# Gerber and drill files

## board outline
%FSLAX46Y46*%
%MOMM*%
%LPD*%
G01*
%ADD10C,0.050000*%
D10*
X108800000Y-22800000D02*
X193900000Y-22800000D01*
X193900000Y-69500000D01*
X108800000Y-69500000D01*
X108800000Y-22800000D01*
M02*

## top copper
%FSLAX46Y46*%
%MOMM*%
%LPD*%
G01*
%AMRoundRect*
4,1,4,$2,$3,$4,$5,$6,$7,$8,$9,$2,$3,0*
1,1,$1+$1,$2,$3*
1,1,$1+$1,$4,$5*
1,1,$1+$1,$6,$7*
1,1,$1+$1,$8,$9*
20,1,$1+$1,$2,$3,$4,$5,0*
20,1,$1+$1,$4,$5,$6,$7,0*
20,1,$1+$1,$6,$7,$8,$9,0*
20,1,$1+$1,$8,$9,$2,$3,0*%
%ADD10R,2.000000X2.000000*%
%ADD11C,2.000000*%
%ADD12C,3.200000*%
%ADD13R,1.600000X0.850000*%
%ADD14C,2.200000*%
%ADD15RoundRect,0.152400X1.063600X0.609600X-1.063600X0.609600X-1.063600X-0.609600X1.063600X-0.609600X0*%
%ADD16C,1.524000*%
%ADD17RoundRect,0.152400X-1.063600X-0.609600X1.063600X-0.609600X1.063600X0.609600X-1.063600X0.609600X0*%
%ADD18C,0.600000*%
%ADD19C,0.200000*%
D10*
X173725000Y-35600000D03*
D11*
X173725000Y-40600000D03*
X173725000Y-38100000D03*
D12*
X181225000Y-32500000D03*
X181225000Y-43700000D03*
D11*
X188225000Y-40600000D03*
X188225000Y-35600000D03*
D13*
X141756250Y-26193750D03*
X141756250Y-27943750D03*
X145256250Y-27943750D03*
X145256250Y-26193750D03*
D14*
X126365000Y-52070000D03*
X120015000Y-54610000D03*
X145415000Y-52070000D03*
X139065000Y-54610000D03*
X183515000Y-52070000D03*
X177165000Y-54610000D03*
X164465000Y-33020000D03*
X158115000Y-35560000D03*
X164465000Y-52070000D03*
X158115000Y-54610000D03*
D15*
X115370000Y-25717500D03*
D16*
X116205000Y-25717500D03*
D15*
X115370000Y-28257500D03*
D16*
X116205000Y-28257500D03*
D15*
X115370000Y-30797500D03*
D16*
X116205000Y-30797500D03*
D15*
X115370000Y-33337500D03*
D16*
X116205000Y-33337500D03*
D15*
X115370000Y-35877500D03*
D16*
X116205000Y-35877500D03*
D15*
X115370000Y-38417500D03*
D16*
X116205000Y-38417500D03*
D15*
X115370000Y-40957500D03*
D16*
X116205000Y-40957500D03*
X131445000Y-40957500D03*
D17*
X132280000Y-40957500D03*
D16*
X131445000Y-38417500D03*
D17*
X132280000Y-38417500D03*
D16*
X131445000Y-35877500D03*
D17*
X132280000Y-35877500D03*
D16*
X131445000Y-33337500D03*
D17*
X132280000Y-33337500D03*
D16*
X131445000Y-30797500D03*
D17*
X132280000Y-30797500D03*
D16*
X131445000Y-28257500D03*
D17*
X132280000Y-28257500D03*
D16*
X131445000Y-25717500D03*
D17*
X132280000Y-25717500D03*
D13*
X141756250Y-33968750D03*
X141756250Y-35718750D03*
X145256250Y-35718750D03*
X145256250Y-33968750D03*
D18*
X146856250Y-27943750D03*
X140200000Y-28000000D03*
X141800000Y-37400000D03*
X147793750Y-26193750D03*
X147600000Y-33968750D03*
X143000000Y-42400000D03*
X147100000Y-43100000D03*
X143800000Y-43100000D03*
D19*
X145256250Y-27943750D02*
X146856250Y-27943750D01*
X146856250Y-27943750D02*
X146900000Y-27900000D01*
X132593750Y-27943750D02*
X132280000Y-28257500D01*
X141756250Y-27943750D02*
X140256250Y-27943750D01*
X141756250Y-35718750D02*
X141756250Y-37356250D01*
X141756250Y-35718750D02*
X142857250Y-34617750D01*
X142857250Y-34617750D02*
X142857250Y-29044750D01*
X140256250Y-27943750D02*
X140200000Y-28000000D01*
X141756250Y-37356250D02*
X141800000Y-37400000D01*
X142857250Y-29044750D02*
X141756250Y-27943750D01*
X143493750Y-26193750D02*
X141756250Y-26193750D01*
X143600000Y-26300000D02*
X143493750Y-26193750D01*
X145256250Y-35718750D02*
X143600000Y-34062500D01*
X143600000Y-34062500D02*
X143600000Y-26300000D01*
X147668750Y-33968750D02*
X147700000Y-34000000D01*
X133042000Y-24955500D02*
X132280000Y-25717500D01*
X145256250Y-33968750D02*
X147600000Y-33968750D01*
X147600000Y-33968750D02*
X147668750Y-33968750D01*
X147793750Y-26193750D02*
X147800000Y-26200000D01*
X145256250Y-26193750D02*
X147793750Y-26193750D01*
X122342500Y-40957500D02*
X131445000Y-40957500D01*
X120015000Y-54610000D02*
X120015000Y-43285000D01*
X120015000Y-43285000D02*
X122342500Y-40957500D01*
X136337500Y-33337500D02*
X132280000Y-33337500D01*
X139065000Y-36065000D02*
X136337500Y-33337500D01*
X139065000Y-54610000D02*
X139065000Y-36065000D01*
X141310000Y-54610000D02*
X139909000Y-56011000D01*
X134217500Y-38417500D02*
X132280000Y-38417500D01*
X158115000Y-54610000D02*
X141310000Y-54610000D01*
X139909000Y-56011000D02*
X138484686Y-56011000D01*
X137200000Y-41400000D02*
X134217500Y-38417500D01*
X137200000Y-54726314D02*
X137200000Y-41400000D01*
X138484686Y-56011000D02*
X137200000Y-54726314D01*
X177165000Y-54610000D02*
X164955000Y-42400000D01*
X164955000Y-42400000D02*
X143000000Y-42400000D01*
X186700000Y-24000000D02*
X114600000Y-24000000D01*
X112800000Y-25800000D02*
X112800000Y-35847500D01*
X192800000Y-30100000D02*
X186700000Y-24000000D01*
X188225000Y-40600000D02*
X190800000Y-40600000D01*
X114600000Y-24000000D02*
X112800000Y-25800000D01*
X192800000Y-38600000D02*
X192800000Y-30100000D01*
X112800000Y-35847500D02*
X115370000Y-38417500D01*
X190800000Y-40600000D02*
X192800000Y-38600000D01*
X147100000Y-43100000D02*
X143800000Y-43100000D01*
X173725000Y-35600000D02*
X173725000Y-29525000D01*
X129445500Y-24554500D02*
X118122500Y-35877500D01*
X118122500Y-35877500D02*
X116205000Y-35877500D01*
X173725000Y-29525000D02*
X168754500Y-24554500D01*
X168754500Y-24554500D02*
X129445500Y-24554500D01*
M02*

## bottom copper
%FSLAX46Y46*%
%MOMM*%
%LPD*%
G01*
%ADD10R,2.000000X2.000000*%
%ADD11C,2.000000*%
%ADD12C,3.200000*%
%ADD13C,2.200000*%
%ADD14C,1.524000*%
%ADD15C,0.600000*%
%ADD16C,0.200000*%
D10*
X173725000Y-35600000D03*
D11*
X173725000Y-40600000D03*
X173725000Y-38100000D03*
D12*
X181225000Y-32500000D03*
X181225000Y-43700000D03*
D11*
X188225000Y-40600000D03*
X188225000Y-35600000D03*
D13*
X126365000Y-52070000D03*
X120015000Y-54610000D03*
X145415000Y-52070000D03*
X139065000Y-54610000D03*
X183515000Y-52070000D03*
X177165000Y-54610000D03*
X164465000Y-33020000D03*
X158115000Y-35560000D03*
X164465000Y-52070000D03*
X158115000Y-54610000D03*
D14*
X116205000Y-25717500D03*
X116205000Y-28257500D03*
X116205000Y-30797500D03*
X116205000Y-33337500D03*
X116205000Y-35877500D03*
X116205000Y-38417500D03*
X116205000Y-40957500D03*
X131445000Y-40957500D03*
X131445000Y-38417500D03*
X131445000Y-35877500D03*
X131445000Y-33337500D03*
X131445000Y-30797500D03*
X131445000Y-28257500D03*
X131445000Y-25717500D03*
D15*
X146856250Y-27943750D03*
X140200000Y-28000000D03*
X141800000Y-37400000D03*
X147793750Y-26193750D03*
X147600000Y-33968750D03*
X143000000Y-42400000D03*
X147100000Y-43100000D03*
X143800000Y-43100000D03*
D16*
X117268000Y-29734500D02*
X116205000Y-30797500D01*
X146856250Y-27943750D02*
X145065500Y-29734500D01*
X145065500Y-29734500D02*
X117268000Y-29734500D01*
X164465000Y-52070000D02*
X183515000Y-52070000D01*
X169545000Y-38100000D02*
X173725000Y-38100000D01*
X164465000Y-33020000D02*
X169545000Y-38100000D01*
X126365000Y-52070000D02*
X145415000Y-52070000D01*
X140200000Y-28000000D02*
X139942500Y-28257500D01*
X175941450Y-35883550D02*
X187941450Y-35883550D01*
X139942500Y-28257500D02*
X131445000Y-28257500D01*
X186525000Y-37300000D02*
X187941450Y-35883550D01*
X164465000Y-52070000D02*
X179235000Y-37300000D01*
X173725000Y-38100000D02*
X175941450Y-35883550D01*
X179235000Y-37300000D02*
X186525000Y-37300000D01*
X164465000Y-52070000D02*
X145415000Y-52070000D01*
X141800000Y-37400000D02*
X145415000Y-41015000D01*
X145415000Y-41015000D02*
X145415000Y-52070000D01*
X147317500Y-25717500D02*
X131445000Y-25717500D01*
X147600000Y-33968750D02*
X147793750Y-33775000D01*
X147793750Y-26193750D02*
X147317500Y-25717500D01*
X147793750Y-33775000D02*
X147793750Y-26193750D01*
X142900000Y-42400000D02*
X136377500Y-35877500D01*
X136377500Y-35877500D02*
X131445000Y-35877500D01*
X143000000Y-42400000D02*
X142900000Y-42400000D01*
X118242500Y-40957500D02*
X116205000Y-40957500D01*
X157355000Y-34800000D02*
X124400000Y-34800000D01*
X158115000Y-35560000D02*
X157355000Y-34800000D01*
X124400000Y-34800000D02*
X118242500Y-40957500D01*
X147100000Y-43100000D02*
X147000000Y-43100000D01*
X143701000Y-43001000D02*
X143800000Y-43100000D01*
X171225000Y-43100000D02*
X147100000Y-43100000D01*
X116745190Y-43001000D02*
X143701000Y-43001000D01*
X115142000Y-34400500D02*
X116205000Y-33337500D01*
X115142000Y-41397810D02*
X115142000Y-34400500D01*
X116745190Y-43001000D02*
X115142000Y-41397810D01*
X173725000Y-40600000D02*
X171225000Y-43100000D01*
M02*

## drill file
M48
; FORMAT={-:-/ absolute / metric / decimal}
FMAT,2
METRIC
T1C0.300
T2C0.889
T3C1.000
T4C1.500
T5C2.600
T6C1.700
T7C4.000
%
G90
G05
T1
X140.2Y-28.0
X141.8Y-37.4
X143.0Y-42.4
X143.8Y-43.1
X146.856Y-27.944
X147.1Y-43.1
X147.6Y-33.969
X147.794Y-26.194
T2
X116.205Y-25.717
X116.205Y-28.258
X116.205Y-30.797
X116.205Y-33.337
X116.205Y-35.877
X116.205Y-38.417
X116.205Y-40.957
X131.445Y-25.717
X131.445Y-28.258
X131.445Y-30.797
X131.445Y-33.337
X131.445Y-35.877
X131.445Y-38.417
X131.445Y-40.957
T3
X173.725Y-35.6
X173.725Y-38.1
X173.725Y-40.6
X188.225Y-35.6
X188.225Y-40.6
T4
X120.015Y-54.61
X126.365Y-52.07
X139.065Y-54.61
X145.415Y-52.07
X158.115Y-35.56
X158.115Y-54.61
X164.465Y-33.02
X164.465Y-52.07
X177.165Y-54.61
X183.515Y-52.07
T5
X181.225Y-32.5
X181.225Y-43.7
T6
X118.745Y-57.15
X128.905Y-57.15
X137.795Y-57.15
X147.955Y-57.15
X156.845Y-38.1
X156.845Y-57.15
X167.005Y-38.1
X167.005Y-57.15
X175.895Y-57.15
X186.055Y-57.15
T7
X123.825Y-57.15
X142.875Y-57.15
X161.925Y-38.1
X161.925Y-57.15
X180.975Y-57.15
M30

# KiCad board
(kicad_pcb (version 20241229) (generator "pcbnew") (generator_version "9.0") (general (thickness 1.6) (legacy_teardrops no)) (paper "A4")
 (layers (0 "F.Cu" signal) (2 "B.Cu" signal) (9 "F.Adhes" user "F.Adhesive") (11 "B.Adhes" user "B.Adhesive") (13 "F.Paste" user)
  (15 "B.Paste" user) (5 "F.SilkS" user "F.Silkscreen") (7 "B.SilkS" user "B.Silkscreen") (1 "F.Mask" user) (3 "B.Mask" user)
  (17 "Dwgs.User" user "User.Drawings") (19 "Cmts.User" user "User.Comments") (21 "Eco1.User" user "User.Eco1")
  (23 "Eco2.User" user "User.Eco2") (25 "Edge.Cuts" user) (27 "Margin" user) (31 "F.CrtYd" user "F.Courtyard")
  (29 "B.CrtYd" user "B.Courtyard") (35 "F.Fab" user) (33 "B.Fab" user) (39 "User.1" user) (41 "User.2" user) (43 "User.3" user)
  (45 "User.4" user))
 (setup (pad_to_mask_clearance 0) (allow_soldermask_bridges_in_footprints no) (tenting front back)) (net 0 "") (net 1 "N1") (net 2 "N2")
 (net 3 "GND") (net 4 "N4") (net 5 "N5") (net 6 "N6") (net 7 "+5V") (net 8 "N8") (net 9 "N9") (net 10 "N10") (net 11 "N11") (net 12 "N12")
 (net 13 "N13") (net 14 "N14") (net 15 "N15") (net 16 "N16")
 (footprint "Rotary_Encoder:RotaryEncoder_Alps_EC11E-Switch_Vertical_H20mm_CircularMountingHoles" (layer "F.Cu") (at 173.725 35.6)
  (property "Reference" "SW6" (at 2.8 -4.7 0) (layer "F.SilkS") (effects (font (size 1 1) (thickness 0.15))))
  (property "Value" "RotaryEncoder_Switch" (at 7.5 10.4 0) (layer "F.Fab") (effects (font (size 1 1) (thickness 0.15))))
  (pad "A" thru_hole rect (at 0 0) (size 2 2) (drill 1) (layers "*.Cu" "*.Mask") (remove_unused_layers no) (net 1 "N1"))
  (pad "B" thru_hole circle (at 0 5) (size 2 2) (drill 1) (layers "*.Cu" "*.Mask") (remove_unused_layers no) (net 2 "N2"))
  (pad "C" thru_hole circle (at 0 2.5) (size 2 2) (drill 1) (layers "*.Cu" "*.Mask") (remove_unused_layers no) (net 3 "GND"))
  (pad "MP" thru_hole circle (at 7.5 -3.1) (size 3.2 3.2) (drill 2.6) (layers "*.Cu" "*.Mask") (remove_unused_layers no))
  (pad "MP" thru_hole circle (at 7.5 8.1) (size 3.2 3.2) (drill 2.6) (layers "*.Cu" "*.Mask") (remove_unused_layers no))
  (pad "S1" thru_hole circle (at 14.5 5) (size 2 2) (drill 1) (layers "*.Cu" "*.Mask") (remove_unused_layers no) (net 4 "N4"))
  (pad "S2" thru_hole circle (at 14.5 0) (size 2 2) (drill 1) (layers "*.Cu" "*.Mask") (remove_unused_layers no) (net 3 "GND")))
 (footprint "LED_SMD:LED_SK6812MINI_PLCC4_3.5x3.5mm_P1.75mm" (layer "F.Cu") (at 143.50625 27.06875)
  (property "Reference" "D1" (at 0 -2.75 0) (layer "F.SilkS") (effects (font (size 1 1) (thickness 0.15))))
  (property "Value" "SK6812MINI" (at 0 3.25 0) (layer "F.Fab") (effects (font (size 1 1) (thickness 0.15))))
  (pad "1" smd rect (at -1.75 -0.875) (size 1.6 0.85) (layers "F.Cu" "F.Mask" "F.Paste") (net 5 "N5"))
  (pad "2" smd rect (at -1.75 0.875) (size 1.6 0.85) (layers "F.Cu" "F.Mask" "F.Paste") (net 3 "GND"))
  (pad "3" smd rect (at 1.75 0.875) (size 1.6 0.85) (layers "F.Cu" "F.Mask" "F.Paste") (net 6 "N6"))
  (pad "4" smd rect (at 1.75 -0.875) (size 1.6 0.85) (layers "F.Cu" "F.Mask" "F.Paste") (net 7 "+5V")))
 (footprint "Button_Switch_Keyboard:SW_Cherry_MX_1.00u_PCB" (layer "F.Cu") (at 126.365 52.07)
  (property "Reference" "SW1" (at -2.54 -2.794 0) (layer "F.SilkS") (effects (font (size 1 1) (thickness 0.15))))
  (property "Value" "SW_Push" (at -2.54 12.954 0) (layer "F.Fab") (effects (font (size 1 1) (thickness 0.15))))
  (pad "" np_thru_hole circle (at -7.62 5.08) (size 1.7 1.7) (drill 1.7) (layers "*.Cu" "*.Mask"))
  (pad "" np_thru_hole circle (at -2.54 5.08) (size 4 4) (drill 4) (layers "*.Cu" "*.Mask"))
  (pad "" np_thru_hole circle (at 2.54 5.08) (size 1.7 1.7) (drill 1.7) (layers "*.Cu" "*.Mask"))
  (pad "1" thru_hole circle (at 0 0) (size 2.2 2.2) (drill 1.5) (layers "*.Cu" "*.Mask") (remove_unused_layers no) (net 3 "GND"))
  (pad "2" thru_hole circle (at -6.35 2.54) (size 2.2 2.2) (drill 1.5) (layers "*.Cu" "*.Mask") (remove_unused_layers no) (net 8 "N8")))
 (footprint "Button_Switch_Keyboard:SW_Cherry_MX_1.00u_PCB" (layer "F.Cu") (at 145.415 52.07)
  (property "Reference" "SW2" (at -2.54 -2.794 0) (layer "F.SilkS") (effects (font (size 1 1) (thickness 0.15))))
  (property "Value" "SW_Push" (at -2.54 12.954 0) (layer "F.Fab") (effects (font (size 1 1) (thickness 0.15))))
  (pad "" np_thru_hole circle (at -7.62 5.08) (size 1.7 1.7) (drill 1.7) (layers "*.Cu" "*.Mask"))
  (pad "" np_thru_hole circle (at -2.54 5.08) (size 4 4) (drill 4) (layers "*.Cu" "*.Mask"))
  (pad "" np_thru_hole circle (at 2.54 5.08) (size 1.7 1.7) (drill 1.7) (layers "*.Cu" "*.Mask"))
  (pad "1" thru_hole circle (at 0 0) (size 2.2 2.2) (drill 1.5) (layers "*.Cu" "*.Mask") (remove_unused_layers no) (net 3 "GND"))
  (pad "2" thru_hole circle (at -6.35 2.54) (size 2.2 2.2) (drill 1.5) (layers "*.Cu" "*.Mask") (remove_unused_layers no) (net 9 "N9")))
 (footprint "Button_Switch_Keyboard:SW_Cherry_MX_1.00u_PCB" (layer "F.Cu") (at 183.515 52.07)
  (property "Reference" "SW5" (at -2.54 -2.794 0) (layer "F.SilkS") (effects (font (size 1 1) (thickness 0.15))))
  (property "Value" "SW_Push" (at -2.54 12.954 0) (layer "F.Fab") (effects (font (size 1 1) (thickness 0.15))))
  (pad "" np_thru_hole circle (at -7.62 5.08) (size 1.7 1.7) (drill 1.7) (layers "*.Cu" "*.Mask"))
  (pad "" np_thru_hole circle (at -2.54 5.08) (size 4 4) (drill 4) (layers "*.Cu" "*.Mask"))
  (pad "" np_thru_hole circle (at 2.54 5.08) (size 1.7 1.7) (drill 1.7) (layers "*.Cu" "*.Mask"))
  (pad "1" thru_hole circle (at 0 0) (size 2.2 2.2) (drill 1.5) (layers "*.Cu" "*.Mask") (remove_unused_layers no) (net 3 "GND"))
  (pad "2" thru_hole circle (at -6.35 2.54) (size 2.2 2.2) (drill 1.5) (layers "*.Cu" "*.Mask") (remove_unused_layers no) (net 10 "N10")))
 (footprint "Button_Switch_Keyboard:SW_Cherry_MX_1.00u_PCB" (layer "F.Cu") (at 164.465 33.02)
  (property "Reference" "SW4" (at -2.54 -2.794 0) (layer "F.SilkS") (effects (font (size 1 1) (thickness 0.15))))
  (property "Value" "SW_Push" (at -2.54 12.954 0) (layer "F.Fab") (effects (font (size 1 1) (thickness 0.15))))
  (pad "" np_thru_hole circle (at -7.62 5.08) (size 1.7 1.7) (drill 1.7) (layers "*.Cu" "*.Mask"))
  (pad "" np_thru_hole circle (at -2.54 5.08) (size 4 4) (drill 4) (layers "*.Cu" "*.Mask"))
  (pad "" np_thru_hole circle (at 2.54 5.08) (size 1.7 1.7) (drill 1.7) (layers "*.Cu" "*.Mask"))
  (pad "1" thru_hole circle (at 0 0) (size 2.2 2.2) (drill 1.5) (layers "*.Cu" "*.Mask") (remove_unused_layers no) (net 3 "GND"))
  (pad "2" thru_hole circle (at -6.35 2.54) (size 2.2 2.2) (drill 1.5) (layers "*.Cu" "*.Mask") (remove_unused_layers no) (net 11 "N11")))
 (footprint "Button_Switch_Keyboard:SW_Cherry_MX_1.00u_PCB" (layer "F.Cu") (at 164.465 52.07)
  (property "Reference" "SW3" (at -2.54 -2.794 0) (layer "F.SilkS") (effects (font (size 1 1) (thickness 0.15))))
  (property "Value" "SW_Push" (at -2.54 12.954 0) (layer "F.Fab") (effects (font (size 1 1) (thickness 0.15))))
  (pad "" np_thru_hole circle (at -7.62 5.08) (size 1.7 1.7) (drill 1.7) (layers "*.Cu" "*.Mask"))
  (pad "" np_thru_hole circle (at -2.54 5.08) (size 4 4) (drill 4) (layers "*.Cu" "*.Mask"))
  (pad "" np_thru_hole circle (at 2.54 5.08) (size 1.7 1.7) (drill 1.7) (layers "*.Cu" "*.Mask"))
  (pad "1" thru_hole circle (at 0 0) (size 2.2 2.2) (drill 1.5) (layers "*.Cu" "*.Mask") (remove_unused_layers no) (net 3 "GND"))
  (pad "2" thru_hole circle (at -6.35 2.54) (size 2.2 2.2) (drill 1.5) (layers "*.Cu" "*.Mask") (remove_unused_layers no) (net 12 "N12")))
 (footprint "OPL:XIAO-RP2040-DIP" (layer "F.Cu") (at 123.825 33.3375)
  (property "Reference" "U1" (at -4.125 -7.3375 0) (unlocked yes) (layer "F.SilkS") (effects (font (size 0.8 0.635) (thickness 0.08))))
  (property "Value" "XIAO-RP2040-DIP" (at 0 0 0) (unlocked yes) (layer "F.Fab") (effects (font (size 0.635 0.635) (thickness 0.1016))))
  (pad "1" smd roundrect (at -8.455 -7.62 180) (size 2.432 1.524) (layers "F.Cu" "F.Mask") (roundrect_rratio 0.1) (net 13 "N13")
   (thermal_bridge_angle 45))
  (pad "1" thru_hole circle (at -7.62 -7.62 180) (size 1.524 1.524) (drill 0.889) (layers "*.Cu" "*.Mask") (remove_unused_layers no)
   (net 13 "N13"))
  (pad "2" smd roundrect (at -8.455 -5.08 180) (size 2.432 1.524) (layers "F.Cu" "F.Mask") (roundrect_rratio 0.1) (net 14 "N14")
   (thermal_bridge_angle 45))
  (pad "2" thru_hole circle (at -7.62 -5.08 180) (size 1.524 1.524) (drill 0.889) (layers "*.Cu" "*.Mask") (remove_unused_layers no)
   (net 14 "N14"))
  (pad "3" smd roundrect (at -8.455 -2.54 180) (size 2.432 1.524) (layers "F.Cu" "F.Mask") (roundrect_rratio 0.1) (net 6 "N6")
   (thermal_bridge_angle 45))
  (pad "3" thru_hole circle (at -7.62 -2.54 180) (size 1.524 1.524) (drill 0.889) (layers "*.Cu" "*.Mask") (remove_unused_layers no)
   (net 6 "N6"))
  (pad "4" smd roundrect (at -8.455 0 180) (size 2.432 1.524) (layers "F.Cu" "F.Mask") (roundrect_rratio 0.1) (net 2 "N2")
   (thermal_bridge_angle 45))
  (pad "4" thru_hole circle (at -7.62 0 180) (size 1.524 1.524) (drill 0.889) (layers "*.Cu" "*.Mask") (remove_unused_layers no)
   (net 2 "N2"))
  (pad "5" smd roundrect (at -8.455 2.54 180) (size 2.432 1.524) (layers "F.Cu" "F.Mask") (roundrect_rratio 0.1) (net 1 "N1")
   (thermal_bridge_angle 45))
  (pad "5" thru_hole circle (at -7.62 2.54 180) (size 1.524 1.524) (drill 0.889) (layers "*.Cu" "*.Mask") (remove_unused_layers no)
   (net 1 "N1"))
  (pad "6" smd roundrect (at -8.455 5.08 180) (size 2.432 1.524) (layers "F.Cu" "F.Mask") (roundrect_rratio 0.1) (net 4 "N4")
   (thermal_bridge_angle 45))
  (pad "6" thru_hole circle (at -7.62 5.08 180) (size 1.524 1.524) (drill 0.889) (layers "*.Cu" "*.Mask") (remove_unused_layers no)
   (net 4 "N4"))
  (pad "7" smd roundrect (at -8.455 7.62 180) (size 2.432 1.524) (layers "F.Cu" "F.Mask") (roundrect_rratio 0.1) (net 11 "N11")
   (thermal_bridge_angle 45))
  (pad "7" thru_hole circle (at -7.62 7.62 180) (size 1.524 1.524) (drill 0.889) (layers "*.Cu" "*.Mask") (remove_unused_layers no)
   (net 11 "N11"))
  (pad "8" thru_hole circle (at 7.62 7.62) (size 1.524 1.524) (drill 0.889) (layers "*.Cu" "*.Mask") (remove_unused_layers no) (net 8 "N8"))
  (pad "8" smd roundrect (at 8.455 7.62) (size 2.432 1.524) (layers "F.Cu" "F.Mask") (roundrect_rratio 0.1) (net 8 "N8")
   (thermal_bridge_angle 45))
  (pad "9" thru_hole circle (at 7.62 5.08) (size 1.524 1.524) (drill 0.889) (layers "*.Cu" "*.Mask") (remove_unused_layers no)
   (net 12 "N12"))
  (pad "9" smd roundrect (at 8.455 5.08) (size 2.432 1.524) (layers "F.Cu" "F.Mask") (roundrect_rratio 0.1) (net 12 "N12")
   (thermal_bridge_angle 45))
  (pad "10" thru_hole circle (at 7.62 2.54) (size 1.524 1.524) (drill 0.889) (layers "*.Cu" "*.Mask") (remove_unused_layers no)
   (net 10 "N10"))
  (pad "10" smd roundrect (at 8.455 2.54) (size 2.432 1.524) (layers "F.Cu" "F.Mask") (roundrect_rratio 0.1) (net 10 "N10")
   (thermal_bridge_angle 45))
  (pad "11" thru_hole circle (at 7.62 0) (size 1.524 1.524) (drill 0.889) (layers "*.Cu" "*.Mask") (remove_unused_layers no) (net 9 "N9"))
  (pad "11" smd roundrect (at 8.455 0) (size 2.432 1.524) (layers "F.Cu" "F.Mask") (roundrect_rratio 0.1) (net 9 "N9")
   (thermal_bridge_angle 45))
  (pad "12" thru_hole circle (at 7.62 -2.54) (size 1.524 1.524) (drill 0.889) (layers "*.Cu" "*.Mask") (remove_unused_layers no)
   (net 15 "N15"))
  (pad "12" smd roundrect (at 8.455 -2.54) (size 2.432 1.524) (layers "F.Cu" "F.Mask") (roundrect_rratio 0.1) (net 15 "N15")
   (thermal_bridge_angle 45))
  (pad "13" thru_hole circle (at 7.62 -5.08) (size 1.524 1.524) (drill 0.889) (layers "*.Cu" "*.Mask") (remove_unused_layers no)
   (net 3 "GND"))
  (pad "13" smd roundrect (at 8.455 -5.08) (size 2.432 1.524) (layers "F.Cu" "F.Mask") (roundrect_rratio 0.1) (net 3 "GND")
   (thermal_bridge_angle 45))
  (pad "14" thru_hole circle (at 7.62 -7.62) (size 1.524 1.524) (drill 0.889) (layers "*.Cu" "*.Mask") (remove_unused_layers no)
   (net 7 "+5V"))
  (pad "14" smd roundrect (at 8.455 -7.62) (size 2.432 1.524) (layers "F.Cu" "F.Mask") (roundrect_rratio 0.1) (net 7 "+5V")
   (thermal_bridge_angle 45)))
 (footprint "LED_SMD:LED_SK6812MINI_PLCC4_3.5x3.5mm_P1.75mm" (layer "F.Cu") (at 143.50625 34.84375)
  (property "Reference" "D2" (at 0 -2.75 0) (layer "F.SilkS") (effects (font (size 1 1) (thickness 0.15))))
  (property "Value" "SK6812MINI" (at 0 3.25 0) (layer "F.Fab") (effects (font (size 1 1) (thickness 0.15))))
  (pad "1" smd rect (at -1.75 -0.875) (size 1.6 0.85) (layers "F.Cu" "F.Mask" "F.Paste") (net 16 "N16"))
  (pad "2" smd rect (at -1.75 0.875) (size 1.6 0.85) (layers "F.Cu" "F.Mask" "F.Paste") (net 3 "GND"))
  (pad "3" smd rect (at 1.75 0.875) (size 1.6 0.85) (layers "F.Cu" "F.Mask" "F.Paste") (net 5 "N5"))
  (pad "4" smd rect (at 1.75 -0.875) (size 1.6 0.85) (layers "F.Cu" "F.Mask" "F.Paste") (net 7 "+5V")))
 (gr_rect (start 108.8 22.8) (end 193.9 69.5) (stroke (width 0.05) (type default)) (fill no) (layer "Edge.Cuts"))
 (segment (start 145.25625 27.94375) (end 146.85625 27.94375) (width 0.2) (layer "F.Cu") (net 6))
 (segment (start 146.85625 27.94375) (end 146.9 27.9) (width 0.2) (layer "F.Cu") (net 6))
 (via (at 146.85625 27.94375) (size 0.6) (drill 0.3) (layers "F.Cu" "B.Cu") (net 6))
 (segment (start 117.268 29.7345) (end 116.205 30.7975) (width 0.2) (layer "B.Cu") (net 6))
 (segment (start 146.85625 27.94375) (end 145.0655 29.7345) (width 0.2) (layer "B.Cu") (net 6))
 (segment (start 145.0655 29.7345) (end 117.268 29.7345) (width 0.2) (layer "B.Cu") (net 6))
 (segment (start 132.59375 27.94375) (end 132.28 28.2575) (width 0.2) (layer "F.Cu") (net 3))
 (segment (start 141.75625 27.94375) (end 140.25625 27.94375) (width 0.2) (layer "F.Cu") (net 3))
 (segment (start 141.75625 35.71875) (end 141.75625 37.35625) (width 0.2) (layer "F.Cu") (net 3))
 (segment (start 141.75625 35.71875) (end 142.85725 34.61775) (width 0.2) (layer "F.Cu") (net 3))
 (segment (start 142.85725 34.61775) (end 142.85725 29.04475) (width 0.2) (layer "F.Cu") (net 3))
 (segment (start 140.25625 27.94375) (end 140.2 28) (width 0.2) (layer "F.Cu") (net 3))
 (segment (start 141.75625 37.35625) (end 141.8 37.4) (width 0.2) (layer "F.Cu") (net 3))
 (segment (start 142.85725 29.04475) (end 141.75625 27.94375) (width 0.2) (layer "F.Cu") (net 3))
 (via (at 140.2 28) (size 0.6) (drill 0.3) (layers "F.Cu" "B.Cu") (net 3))
 (via (at 141.8 37.4) (size 0.6) (drill 0.3) (layers "F.Cu" "B.Cu") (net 3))
 (segment (start 164.465 52.07) (end 183.515 52.07) (width 0.2) (layer "B.Cu") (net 3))
 (segment (start 169.545 38.1) (end 173.725 38.1) (width 0.2) (layer "B.Cu") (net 3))
 (segment (start 164.465 33.02) (end 169.545 38.1) (width 0.2) (layer "B.Cu") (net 3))
 (segment (start 126.365 52.07) (end 145.415 52.07) (width 0.2) (layer "B.Cu") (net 3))
 (segment (start 140.2 28) (end 139.9425 28.2575) (width 0.2) (layer "B.Cu") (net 3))
 (segment (start 175.94145 35.88355) (end 187.94145 35.88355) (width 0.2) (layer "B.Cu") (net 3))
 (segment (start 139.9425 28.2575) (end 131.445 28.2575) (width 0.2) (layer "B.Cu") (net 3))
 (segment (start 186.525 37.3) (end 187.94145 35.88355) (width 0.2) (layer "B.Cu") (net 3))
 (segment (start 164.465 52.07) (end 179.235 37.3) (width 0.2) (layer "B.Cu") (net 3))
 (segment (start 173.725 38.1) (end 175.94145 35.88355) (width 0.2) (layer "B.Cu") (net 3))
 (segment (start 179.235 37.3) (end 186.525 37.3) (width 0.2) (layer "B.Cu") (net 3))
 (segment (start 164.465 52.07) (end 145.415 52.07) (width 0.2) (layer "B.Cu") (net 3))
 (segment (start 141.8 37.4) (end 145.415 41.015) (width 0.2) (layer "B.Cu") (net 3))
 (segment (start 145.415 41.015) (end 145.415 52.07) (width 0.2) (layer "B.Cu") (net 3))
 (segment (start 143.49375 26.19375) (end 141.75625 26.19375) (width 0.2) (layer "F.Cu") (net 5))
 (segment (start 143.6 26.3) (end 143.49375 26.19375) (width 0.2) (layer "F.Cu") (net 5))
 (segment (start 145.25625 35.71875) (end 143.6 34.0625) (width 0.2) (layer "F.Cu") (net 5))
 (segment (start 143.6 34.0625) (end 143.6 26.3) (width 0.2) (layer "F.Cu") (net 5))
 (segment (start 147.66875 33.96875) (end 147.7 34) (width 0.2) (layer "F.Cu") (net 7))
 (segment (start 133.042 24.9555) (end 132.28 25.7175) (width 0.2) (layer "F.Cu") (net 7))
 (segment (start 145.25625 33.96875) (end 147.6 33.96875) (width 0.2) (layer "F.Cu") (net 7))
 (segment (start 147.6 33.96875) (end 147.66875 33.96875) (width 0.2) (layer "F.Cu") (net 7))
 (segment (start 147.79375 26.19375) (end 147.8 26.2) (width 0.2) (layer "F.Cu") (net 7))
 (segment (start 145.25625 26.19375) (end 147.79375 26.19375) (width 0.2) (layer "F.Cu") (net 7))
 (via (at 147.79375 26.19375) (size 0.6) (drill 0.3) (layers "F.Cu" "B.Cu") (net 7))
 (via (at 147.6 33.96875) (size 0.6) (drill 0.3) (layers "F.Cu" "B.Cu") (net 7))
 (segment (start 147.3175 25.7175) (end 131.445 25.7175) (width 0.2) (layer "B.Cu") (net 7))
 (segment (start 147.6 33.96875) (end 147.79375 33.775) (width 0.2) (layer "B.Cu") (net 7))
 (segment (start 147.79375 26.19375) (end 147.3175 25.7175) (width 0.2) (layer "B.Cu") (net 7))
 (segment (start 147.79375 33.775) (end 147.79375 26.19375) (width 0.2) (layer "B.Cu") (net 7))
 (segment (start 122.3425 40.9575) (end 131.445 40.9575) (width 0.2) (layer "F.Cu") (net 8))
 (segment (start 120.015 54.61) (end 120.015 43.285) (width 0.2) (layer "F.Cu") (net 8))
 (segment (start 120.015 43.285) (end 122.3425 40.9575) (width 0.2) (layer "F.Cu") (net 8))
 (segment (start 136.3375 33.3375) (end 132.28 33.3375) (width 0.2) (layer "F.Cu") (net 9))
 (segment (start 139.065 36.065) (end 136.3375 33.3375) (width 0.2) (layer "F.Cu") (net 9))
 (segment (start 139.065 54.61) (end 139.065 36.065) (width 0.2) (layer "F.Cu") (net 9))
 (segment (start 141.31 54.61) (end 139.909 56.011) (width 0.2) (layer "F.Cu") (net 12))
 (segment (start 134.2175 38.4175) (end 132.28 38.4175) (width 0.2) (layer "F.Cu") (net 12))
 (segment (start 158.115 54.61) (end 141.31 54.61) (width 0.2) (layer "F.Cu") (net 12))
 (segment (start 139.909 56.011) (end 138.484686 56.011) (width 0.2) (layer "F.Cu") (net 12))
 (segment (start 137.2 41.4) (end 134.2175 38.4175) (width 0.2) (layer "F.Cu") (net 12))
 (segment (start 137.2 54.726314) (end 137.2 41.4) (width 0.2) (layer "F.Cu") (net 12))
 (segment (start 138.484686 56.011) (end 137.2 54.726314) (width 0.2) (layer "F.Cu") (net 12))
 (segment (start 177.165 54.61) (end 164.955 42.4) (width 0.2) (layer "F.Cu") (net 10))
 (segment (start 164.955 42.4) (end 143 42.4) (width 0.2) (layer "F.Cu") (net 10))
 (via (at 143 42.4) (size 0.6) (drill 0.3) (layers "F.Cu" "B.Cu") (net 10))
 (segment (start 142.9 42.4) (end 136.3775 35.8775) (width 0.2) (layer "B.Cu") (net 10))
 (segment (start 136.3775 35.8775) (end 131.445 35.8775) (width 0.2) (layer "B.Cu") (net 10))
 (segment (start 143 42.4) (end 142.9 42.4) (width 0.2) (layer "B.Cu") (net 10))
 (segment (start 118.2425 40.9575) (end 116.205 40.9575) (width 0.2) (layer "B.Cu") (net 11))
 (segment (start 157.355 34.8) (end 124.4 34.8) (width 0.2) (layer "B.Cu") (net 11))
 (segment (start 158.115 35.56) (end 157.355 34.8) (width 0.2) (layer "B.Cu") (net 11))
 (segment (start 124.4 34.8) (end 118.2425 40.9575) (width 0.2) (layer "B.Cu") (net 11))
 (segment (start 186.7 24) (end 114.6 24) (width 0.2) (layer "F.Cu") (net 4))
 (segment (start 112.8 25.8) (end 112.8 35.8475) (width 0.2) (layer "F.Cu") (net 4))
 (segment (start 192.8 30.1) (end 186.7 24) (width 0.2) (layer "F.Cu") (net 4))
 (segment (start 188.225 40.6) (end 190.8 40.6) (width 0.2) (layer "F.Cu") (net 4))
 (segment (start 114.6 24) (end 112.8 25.8) (width 0.2) (layer "F.Cu") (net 4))
 (segment (start 192.8 38.6) (end 192.8 30.1) (width 0.2) (layer "F.Cu") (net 4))
 (segment (start 112.8 35.8475) (end 115.37 38.4175) (width 0.2) (layer "F.Cu") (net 4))
 (segment (start 190.8 40.6) (end 192.8 38.6) (width 0.2) (layer "F.Cu") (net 4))
 (segment (start 147.1 43.1) (end 143.8 43.1) (width 0.2) (layer "F.Cu") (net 2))
 (via (at 147.1 43.1) (size 0.6) (drill 0.3) (layers "F.Cu" "B.Cu") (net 2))
 (via (at 143.8 43.1) (size 0.6) (drill 0.3) (layers "F.Cu" "B.Cu") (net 2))
 (segment (start 147.1 43.1) (end 147 43.1) (width 0.2) (layer "B.Cu") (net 2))
 (segment (start 143.701 43.001) (end 143.8 43.1) (width 0.2) (layer "B.Cu") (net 2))
 (segment (start 171.225 43.1) (end 147.1 43.1) (width 0.2) (layer "B.Cu") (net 2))
 (segment (start 116.74519 43.001) (end 143.701 43.001) (width 0.2) (layer "B.Cu") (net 2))
 (segment (start 115.142 34.4005) (end 116.205 33.3375) (width 0.2) (layer "B.Cu") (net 2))
 (segment (start 115.142 41.39781) (end 115.142 34.4005) (width 0.2) (layer "B.Cu") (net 2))
 (segment (start 116.74519 43.001) (end 115.142 41.39781) (width 0.2) (layer "B.Cu") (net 2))
 (segment (start 173.725 40.6) (end 171.225 43.1) (width 0.2) (layer "B.Cu") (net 2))
 (segment (start 173.725 35.6) (end 173.725 29.525) (width 0.2) (layer "F.Cu") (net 1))
 (segment (start 129.4455 24.5545) (end 118.1225 35.8775) (width 0.2) (layer "F.Cu") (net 1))
 (segment (start 118.1225 35.8775) (end 116.205 35.8775) (width 0.2) (layer "F.Cu") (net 1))
 (segment (start 173.725 29.525) (end 168.7545 24.5545) (width 0.2) (layer "F.Cu") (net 1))
 (segment (start 168.7545 24.5545) (end 129.4455 24.5545) (width 0.2) (layer "F.Cu") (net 1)))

